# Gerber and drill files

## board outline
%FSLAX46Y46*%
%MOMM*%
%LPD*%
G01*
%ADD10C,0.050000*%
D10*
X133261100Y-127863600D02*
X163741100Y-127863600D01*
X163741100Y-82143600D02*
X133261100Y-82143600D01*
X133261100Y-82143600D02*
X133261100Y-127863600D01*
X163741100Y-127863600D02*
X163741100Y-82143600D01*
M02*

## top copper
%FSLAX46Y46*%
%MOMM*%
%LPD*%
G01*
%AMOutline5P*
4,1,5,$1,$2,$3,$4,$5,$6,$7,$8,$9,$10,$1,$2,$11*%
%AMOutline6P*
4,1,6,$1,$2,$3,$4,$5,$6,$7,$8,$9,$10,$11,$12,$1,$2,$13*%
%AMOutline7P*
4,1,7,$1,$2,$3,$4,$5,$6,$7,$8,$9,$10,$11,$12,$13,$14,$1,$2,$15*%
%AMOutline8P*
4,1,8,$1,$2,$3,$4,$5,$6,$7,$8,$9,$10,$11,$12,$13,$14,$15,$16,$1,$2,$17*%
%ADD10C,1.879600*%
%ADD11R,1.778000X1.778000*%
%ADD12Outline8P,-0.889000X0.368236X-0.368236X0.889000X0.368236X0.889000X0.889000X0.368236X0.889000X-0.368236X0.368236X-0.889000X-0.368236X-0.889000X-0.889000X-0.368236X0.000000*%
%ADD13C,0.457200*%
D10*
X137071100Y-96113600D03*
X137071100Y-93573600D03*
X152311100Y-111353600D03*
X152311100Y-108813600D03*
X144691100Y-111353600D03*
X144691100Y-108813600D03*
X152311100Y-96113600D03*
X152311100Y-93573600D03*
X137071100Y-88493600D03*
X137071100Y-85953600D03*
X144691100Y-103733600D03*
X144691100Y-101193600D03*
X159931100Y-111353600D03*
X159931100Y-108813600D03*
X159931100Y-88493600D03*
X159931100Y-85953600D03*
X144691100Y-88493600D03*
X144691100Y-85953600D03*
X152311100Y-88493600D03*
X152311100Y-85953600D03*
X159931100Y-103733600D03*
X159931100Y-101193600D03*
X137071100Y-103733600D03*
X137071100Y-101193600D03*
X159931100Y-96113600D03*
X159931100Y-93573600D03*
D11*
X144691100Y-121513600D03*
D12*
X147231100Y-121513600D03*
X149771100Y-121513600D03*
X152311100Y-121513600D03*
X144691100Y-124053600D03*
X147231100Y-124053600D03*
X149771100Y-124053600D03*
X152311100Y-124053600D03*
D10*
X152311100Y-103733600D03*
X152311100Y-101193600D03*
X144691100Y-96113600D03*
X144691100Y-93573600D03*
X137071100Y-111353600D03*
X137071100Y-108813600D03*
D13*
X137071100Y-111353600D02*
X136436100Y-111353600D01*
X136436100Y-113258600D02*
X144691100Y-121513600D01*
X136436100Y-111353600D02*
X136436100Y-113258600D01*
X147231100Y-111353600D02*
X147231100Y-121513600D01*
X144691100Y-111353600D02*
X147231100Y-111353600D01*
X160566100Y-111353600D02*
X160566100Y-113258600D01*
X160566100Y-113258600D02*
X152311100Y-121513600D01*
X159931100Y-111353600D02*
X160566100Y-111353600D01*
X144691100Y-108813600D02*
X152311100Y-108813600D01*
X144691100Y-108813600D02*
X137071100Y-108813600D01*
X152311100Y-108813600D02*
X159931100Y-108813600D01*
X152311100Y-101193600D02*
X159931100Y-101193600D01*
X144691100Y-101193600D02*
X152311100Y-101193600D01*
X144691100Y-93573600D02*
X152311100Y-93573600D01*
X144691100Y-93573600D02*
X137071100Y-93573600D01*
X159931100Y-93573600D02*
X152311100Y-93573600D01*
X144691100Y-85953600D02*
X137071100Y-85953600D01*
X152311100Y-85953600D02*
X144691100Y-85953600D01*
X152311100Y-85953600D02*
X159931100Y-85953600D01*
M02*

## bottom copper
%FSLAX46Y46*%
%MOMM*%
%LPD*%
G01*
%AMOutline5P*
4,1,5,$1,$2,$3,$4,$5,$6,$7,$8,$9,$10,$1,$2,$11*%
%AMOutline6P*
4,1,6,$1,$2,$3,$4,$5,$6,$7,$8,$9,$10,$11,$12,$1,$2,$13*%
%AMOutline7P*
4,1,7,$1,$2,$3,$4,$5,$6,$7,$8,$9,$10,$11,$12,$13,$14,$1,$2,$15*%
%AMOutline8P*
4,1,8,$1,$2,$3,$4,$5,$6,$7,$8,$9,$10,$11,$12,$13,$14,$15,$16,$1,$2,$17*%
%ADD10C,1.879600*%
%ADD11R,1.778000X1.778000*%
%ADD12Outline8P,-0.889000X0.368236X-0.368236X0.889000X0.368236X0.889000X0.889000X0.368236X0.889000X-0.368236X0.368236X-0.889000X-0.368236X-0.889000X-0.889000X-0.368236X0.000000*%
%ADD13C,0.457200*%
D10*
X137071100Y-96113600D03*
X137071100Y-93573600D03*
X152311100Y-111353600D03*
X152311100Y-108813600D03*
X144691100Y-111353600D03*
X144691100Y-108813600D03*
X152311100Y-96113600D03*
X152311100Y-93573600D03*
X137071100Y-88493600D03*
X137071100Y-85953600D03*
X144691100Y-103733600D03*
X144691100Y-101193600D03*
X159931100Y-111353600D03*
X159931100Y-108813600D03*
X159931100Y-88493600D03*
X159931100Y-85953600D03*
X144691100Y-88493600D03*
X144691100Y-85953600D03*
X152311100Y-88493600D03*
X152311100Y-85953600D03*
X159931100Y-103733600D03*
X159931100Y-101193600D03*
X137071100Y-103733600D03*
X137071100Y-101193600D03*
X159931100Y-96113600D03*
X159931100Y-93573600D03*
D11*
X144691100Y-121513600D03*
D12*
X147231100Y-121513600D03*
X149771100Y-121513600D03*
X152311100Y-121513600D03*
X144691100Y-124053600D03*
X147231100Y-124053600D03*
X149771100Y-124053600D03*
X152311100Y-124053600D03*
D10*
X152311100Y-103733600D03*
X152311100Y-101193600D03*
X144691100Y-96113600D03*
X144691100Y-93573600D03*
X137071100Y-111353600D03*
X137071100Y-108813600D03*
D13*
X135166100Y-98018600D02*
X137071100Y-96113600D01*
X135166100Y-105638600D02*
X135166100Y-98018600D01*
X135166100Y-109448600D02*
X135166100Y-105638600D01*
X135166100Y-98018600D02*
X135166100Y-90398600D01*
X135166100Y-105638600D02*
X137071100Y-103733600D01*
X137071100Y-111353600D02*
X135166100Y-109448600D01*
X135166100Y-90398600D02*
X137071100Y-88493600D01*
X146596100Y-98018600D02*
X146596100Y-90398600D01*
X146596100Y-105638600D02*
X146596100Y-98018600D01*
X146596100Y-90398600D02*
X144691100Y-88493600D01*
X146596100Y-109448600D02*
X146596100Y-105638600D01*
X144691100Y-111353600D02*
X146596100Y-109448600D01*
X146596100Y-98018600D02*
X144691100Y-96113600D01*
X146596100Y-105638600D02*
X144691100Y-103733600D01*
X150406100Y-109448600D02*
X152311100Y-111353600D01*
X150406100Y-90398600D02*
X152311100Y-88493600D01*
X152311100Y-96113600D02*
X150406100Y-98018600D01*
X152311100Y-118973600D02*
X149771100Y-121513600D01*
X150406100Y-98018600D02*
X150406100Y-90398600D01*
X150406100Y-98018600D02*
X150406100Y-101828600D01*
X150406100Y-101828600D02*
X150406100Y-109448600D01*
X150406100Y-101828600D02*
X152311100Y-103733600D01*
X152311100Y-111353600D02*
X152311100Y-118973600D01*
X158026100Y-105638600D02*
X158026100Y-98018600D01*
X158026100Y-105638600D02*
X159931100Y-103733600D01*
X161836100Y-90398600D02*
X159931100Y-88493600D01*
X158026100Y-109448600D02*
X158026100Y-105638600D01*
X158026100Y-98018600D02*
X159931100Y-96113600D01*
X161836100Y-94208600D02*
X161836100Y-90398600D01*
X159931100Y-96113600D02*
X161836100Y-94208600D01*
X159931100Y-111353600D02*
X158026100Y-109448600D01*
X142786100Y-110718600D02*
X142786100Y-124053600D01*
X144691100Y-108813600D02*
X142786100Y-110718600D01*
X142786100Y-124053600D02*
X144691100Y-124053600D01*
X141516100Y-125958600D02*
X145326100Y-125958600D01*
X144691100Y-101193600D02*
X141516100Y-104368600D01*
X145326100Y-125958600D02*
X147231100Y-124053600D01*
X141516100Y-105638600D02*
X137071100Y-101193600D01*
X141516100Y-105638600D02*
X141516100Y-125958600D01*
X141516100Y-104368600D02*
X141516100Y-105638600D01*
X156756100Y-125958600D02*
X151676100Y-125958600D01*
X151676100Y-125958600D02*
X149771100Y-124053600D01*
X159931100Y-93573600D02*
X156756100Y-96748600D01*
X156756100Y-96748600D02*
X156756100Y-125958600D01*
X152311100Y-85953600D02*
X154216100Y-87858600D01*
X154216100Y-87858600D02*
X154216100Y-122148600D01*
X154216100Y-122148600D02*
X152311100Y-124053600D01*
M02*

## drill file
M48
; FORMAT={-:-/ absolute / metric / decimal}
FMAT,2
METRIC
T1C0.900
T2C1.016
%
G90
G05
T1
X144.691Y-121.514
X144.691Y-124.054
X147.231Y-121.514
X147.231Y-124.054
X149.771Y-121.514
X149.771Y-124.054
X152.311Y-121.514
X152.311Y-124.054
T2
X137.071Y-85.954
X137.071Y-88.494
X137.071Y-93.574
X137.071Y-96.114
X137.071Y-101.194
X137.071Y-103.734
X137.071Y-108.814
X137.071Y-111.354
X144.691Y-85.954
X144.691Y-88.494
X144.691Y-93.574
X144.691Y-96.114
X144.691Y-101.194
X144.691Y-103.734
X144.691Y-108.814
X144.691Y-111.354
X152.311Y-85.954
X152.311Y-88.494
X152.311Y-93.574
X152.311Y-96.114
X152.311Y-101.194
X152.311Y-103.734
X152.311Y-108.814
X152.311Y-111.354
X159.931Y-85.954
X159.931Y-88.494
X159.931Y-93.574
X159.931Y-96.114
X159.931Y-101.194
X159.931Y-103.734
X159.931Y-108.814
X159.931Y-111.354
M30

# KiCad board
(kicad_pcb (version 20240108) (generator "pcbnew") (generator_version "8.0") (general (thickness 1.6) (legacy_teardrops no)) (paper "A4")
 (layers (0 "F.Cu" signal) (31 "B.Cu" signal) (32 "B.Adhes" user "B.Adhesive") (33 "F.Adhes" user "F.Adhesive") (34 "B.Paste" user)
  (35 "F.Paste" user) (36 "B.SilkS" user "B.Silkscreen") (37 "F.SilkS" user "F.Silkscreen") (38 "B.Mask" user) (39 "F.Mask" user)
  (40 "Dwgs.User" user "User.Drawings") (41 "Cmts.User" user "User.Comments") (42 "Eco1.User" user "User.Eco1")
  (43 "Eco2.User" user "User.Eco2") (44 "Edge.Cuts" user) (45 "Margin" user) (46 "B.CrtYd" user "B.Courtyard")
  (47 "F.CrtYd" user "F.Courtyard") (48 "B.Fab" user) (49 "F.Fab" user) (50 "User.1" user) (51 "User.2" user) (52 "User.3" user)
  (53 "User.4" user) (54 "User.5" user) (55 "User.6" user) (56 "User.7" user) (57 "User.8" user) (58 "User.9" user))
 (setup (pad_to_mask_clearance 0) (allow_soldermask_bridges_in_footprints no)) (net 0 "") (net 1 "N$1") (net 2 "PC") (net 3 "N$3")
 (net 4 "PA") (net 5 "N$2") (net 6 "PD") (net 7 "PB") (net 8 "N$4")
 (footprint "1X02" (layer "F.Cu") (at 137.0711 96.1136 90)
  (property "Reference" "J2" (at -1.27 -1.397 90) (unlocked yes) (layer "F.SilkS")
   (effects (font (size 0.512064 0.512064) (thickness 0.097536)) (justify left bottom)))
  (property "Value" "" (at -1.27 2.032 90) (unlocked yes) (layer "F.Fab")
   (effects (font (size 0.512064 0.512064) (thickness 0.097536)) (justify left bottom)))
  (pad "1" thru_hole circle (at 0 0 180) (size 1.8796 1.8796) (drill 1.016) (layers "*.Cu" "*.Mask") (remove_unused_layers no) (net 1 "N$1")
   (solder_mask_margin 0.1016) (thermal_bridge_angle 0))
  (pad "2" thru_hole circle (at 2.54 0 180) (size 1.8796 1.8796) (drill 1.016) (layers "*.Cu" "*.Mask") (remove_unused_layers no)
   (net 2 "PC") (solder_mask_margin 0.1016) (thermal_bridge_angle 0)))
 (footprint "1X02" (layer "F.Cu") (at 152.3111 111.3536 90)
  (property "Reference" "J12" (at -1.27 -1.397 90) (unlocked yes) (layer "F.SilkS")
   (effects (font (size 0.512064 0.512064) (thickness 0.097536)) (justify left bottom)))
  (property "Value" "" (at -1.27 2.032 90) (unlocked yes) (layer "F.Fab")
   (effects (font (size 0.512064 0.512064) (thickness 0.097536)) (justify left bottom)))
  (pad "1" thru_hole circle (at 0 0 180) (size 1.8796 1.8796) (drill 1.016) (layers "*.Cu" "*.Mask") (remove_unused_layers no) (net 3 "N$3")
   (solder_mask_margin 0.1016) (thermal_bridge_angle 0))
  (pad "2" thru_hole circle (at 2.54 0 180) (size 1.8796 1.8796) (drill 1.016) (layers "*.Cu" "*.Mask") (remove_unused_layers no)
   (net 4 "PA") (solder_mask_margin 0.1016) (thermal_bridge_angle 0)))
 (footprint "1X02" (layer "F.Cu") (at 144.6911 111.3536 90)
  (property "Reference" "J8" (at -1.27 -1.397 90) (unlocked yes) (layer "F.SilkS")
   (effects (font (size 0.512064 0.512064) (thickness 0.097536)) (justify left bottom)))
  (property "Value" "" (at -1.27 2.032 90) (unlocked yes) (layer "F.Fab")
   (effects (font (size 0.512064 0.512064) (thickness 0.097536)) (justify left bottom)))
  (pad "1" thru_hole circle (at 0 0 180) (size 1.8796 1.8796) (drill 1.016) (layers "*.Cu" "*.Mask") (remove_unused_layers no) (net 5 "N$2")
   (solder_mask_margin 0.1016) (thermal_bridge_angle 0))
  (pad "2" thru_hole circle (at 2.54 0 180) (size 1.8796 1.8796) (drill 1.016) (layers "*.Cu" "*.Mask") (remove_unused_layers no)
   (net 4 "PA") (solder_mask_margin 0.1016) (thermal_bridge_angle 0)))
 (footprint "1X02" (layer "F.Cu") (at 152.3111 96.1136 90)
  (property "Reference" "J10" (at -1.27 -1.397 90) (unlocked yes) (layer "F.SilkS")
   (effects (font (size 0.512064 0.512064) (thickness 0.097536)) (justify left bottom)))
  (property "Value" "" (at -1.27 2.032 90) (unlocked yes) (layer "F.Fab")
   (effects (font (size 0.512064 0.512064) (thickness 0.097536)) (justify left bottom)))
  (pad "1" thru_hole circle (at 0 0 180) (size 1.8796 1.8796) (drill 1.016) (layers "*.Cu" "*.Mask") (remove_unused_layers no) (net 3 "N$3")
   (solder_mask_margin 0.1016) (thermal_bridge_angle 0))
  (pad "2" thru_hole circle (at 2.54 0 180) (size 1.8796 1.8796) (drill 1.016) (layers "*.Cu" "*.Mask") (remove_unused_layers no)
   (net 2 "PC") (solder_mask_margin 0.1016) (thermal_bridge_angle 0)))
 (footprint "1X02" (layer "F.Cu") (at 137.0711 88.4936 90)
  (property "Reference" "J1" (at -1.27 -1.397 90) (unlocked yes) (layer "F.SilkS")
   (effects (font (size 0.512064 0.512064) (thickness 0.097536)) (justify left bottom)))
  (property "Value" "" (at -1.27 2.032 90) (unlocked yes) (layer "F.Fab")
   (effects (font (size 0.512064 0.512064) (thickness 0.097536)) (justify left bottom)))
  (pad "1" thru_hole circle (at 0 0 180) (size 1.8796 1.8796) (drill 1.016) (layers "*.Cu" "*.Mask") (remove_unused_layers no) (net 1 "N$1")
   (solder_mask_margin 0.1016) (thermal_bridge_angle 0))
  (pad "2" thru_hole circle (at 2.54 0 180) (size 1.8796 1.8796) (drill 1.016) (layers "*.Cu" "*.Mask") (remove_unused_layers no)
   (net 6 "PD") (solder_mask_margin 0.1016) (thermal_bridge_angle 0)))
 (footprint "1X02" (layer "F.Cu") (at 144.6911 103.7336 90)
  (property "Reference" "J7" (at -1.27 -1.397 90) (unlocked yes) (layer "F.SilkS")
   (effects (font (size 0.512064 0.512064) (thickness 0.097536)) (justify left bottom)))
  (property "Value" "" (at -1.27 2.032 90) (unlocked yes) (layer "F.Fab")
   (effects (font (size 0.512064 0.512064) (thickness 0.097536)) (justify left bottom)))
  (pad "1" thru_hole circle (at 0 0 180) (size 1.8796 1.8796) (drill 1.016) (layers "*.Cu" "*.Mask") (remove_unused_layers no) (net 5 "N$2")
   (solder_mask_margin 0.1016) (thermal_bridge_angle 0))
  (pad "2" thru_hole circle (at 2.54 0 180) (size 1.8796 1.8796) (drill 1.016) (layers "*.Cu" "*.Mask") (remove_unused_layers no)
   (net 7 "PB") (solder_mask_margin 0.1016) (thermal_bridge_angle 0)))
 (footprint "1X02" (layer "F.Cu") (at 159.9311 111.3536 90)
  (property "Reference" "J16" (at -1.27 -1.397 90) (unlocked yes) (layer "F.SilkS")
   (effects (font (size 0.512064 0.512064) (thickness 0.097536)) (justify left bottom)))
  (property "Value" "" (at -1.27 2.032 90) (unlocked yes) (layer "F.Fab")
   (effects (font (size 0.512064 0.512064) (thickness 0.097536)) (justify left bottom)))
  (pad "1" thru_hole circle (at 0 0 180) (size 1.8796 1.8796) (drill 1.016) (layers "*.Cu" "*.Mask") (remove_unused_layers no) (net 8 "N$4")
   (solder_mask_margin 0.1016) (thermal_bridge_angle 0))
  (pad "2" thru_hole circle (at 2.54 0 180) (size 1.8796 1.8796) (drill 1.016) (layers "*.Cu" "*.Mask") (remove_unused_layers no)
   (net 4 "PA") (solder_mask_margin 0.1016) (thermal_bridge_angle 0)))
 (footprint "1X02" (layer "F.Cu") (at 159.9311 88.4936 90)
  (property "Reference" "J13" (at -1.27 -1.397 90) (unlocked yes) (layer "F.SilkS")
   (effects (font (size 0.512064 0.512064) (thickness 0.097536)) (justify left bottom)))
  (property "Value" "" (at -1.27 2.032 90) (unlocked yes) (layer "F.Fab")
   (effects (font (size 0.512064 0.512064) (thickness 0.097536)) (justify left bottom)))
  (pad "1" thru_hole circle (at 0 0 180) (size 1.8796 1.8796) (drill 1.016) (layers "*.Cu" "*.Mask") (remove_unused_layers no) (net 8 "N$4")
   (solder_mask_margin 0.1016) (thermal_bridge_angle 0))
  (pad "2" thru_hole circle (at 2.54 0 180) (size 1.8796 1.8796) (drill 1.016) (layers "*.Cu" "*.Mask") (remove_unused_layers no)
   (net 6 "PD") (solder_mask_margin 0.1016) (thermal_bridge_angle 0)))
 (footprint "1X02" (layer "F.Cu") (at 144.6911 88.4936 90)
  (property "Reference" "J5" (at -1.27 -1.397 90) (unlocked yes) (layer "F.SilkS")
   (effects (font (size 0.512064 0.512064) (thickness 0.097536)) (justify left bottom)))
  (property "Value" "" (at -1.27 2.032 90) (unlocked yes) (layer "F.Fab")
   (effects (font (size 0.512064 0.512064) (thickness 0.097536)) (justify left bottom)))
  (pad "1" thru_hole circle (at 0 0 180) (size 1.8796 1.8796) (drill 1.016) (layers "*.Cu" "*.Mask") (remove_unused_layers no) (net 5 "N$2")
   (solder_mask_margin 0.1016) (thermal_bridge_angle 0))
  (pad "2" thru_hole circle (at 2.54 0 180) (size 1.8796 1.8796) (drill 1.016) (layers "*.Cu" "*.Mask") (remove_unused_layers no)
   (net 6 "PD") (solder_mask_margin 0.1016) (thermal_bridge_angle 0)))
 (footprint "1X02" (layer "F.Cu") (at 152.3111 88.4936 90)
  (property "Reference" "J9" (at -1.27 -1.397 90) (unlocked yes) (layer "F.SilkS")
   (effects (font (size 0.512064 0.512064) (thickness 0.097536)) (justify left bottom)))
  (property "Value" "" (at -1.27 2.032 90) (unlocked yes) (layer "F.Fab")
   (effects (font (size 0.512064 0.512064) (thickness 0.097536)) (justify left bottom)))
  (pad "1" thru_hole circle (at 0 0 180) (size 1.8796 1.8796) (drill 1.016) (layers "*.Cu" "*.Mask") (remove_unused_layers no) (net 3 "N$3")
   (solder_mask_margin 0.1016) (thermal_bridge_angle 0))
  (pad "2" thru_hole circle (at 2.54 0 180) (size 1.8796 1.8796) (drill 1.016) (layers "*.Cu" "*.Mask") (remove_unused_layers no)
   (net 6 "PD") (solder_mask_margin 0.1016) (thermal_bridge_angle 0)))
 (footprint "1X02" (layer "F.Cu") (at 159.9311 103.7336 90)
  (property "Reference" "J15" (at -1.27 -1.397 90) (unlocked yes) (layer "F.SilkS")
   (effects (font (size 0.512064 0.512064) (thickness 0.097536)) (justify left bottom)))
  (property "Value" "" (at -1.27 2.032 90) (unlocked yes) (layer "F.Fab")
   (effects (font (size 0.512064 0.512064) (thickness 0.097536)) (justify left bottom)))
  (pad "1" thru_hole circle (at 0 0 180) (size 1.8796 1.8796) (drill 1.016) (layers "*.Cu" "*.Mask") (remove_unused_layers no) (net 8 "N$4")
   (solder_mask_margin 0.1016) (thermal_bridge_angle 0))
  (pad "2" thru_hole circle (at 2.54 0 180) (size 1.8796 1.8796) (drill 1.016) (layers "*.Cu" "*.Mask") (remove_unused_layers no)
   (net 7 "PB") (solder_mask_margin 0.1016) (thermal_bridge_angle 0)))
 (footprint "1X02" (layer "F.Cu") (at 137.0711 103.7336 90)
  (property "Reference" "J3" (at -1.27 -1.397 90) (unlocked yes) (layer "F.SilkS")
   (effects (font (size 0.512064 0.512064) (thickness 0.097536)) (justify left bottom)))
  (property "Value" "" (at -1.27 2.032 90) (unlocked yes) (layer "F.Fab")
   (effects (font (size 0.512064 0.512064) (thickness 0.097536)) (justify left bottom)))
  (pad "1" thru_hole circle (at 0 0 180) (size 1.8796 1.8796) (drill 1.016) (layers "*.Cu" "*.Mask") (remove_unused_layers no) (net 1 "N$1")
   (solder_mask_margin 0.1016) (thermal_bridge_angle 0))
  (pad "2" thru_hole circle (at 2.54 0 180) (size 1.8796 1.8796) (drill 1.016) (layers "*.Cu" "*.Mask") (remove_unused_layers no)
   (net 7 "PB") (solder_mask_margin 0.1016) (thermal_bridge_angle 0)))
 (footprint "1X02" (layer "F.Cu") (at 159.9311 96.1136 90)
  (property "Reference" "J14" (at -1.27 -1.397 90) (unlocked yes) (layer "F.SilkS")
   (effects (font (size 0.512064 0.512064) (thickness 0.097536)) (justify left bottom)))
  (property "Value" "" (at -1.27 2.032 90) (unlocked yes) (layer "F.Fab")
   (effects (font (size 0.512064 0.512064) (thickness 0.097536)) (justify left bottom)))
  (pad "1" thru_hole circle (at 0 0 180) (size 1.8796 1.8796) (drill 1.016) (layers "*.Cu" "*.Mask") (remove_unused_layers no) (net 8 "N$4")
   (solder_mask_margin 0.1016) (thermal_bridge_angle 0))
  (pad "2" thru_hole circle (at 2.54 0 180) (size 1.8796 1.8796) (drill 1.016) (layers "*.Cu" "*.Mask") (remove_unused_layers no)
   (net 2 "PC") (solder_mask_margin 0.1016) (thermal_bridge_angle 0)))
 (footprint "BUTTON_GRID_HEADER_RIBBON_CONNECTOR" (layer "F.Cu") (at 148.5011 122.7836)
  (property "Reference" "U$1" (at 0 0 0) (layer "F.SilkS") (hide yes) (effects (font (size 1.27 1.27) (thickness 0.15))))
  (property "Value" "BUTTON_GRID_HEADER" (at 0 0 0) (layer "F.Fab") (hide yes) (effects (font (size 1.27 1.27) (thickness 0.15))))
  (pad "P1" thru_hole rect (at -3.81 -1.27) (size 1.778 1.778) (drill 0.9) (layers "*.Cu" "*.Mask") (remove_unused_layers no) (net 1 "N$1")
   (solder_mask_margin 0.1016) (thermal_bridge_angle 0))
  (pad "P2" thru_hole roundrect (at -1.27 -1.27) (size 1.778 1.778) (drill 0.9) (layers "*.Cu" "*.Mask") (remove_unused_layers no)
   (roundrect_rratio 0.25) (chamfer_ratio 0.2928932188) (chamfer top_left top_right bottom_left bottom_right) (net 5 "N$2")
   (solder_mask_margin 0.1016) (thermal_bridge_angle 0))
  (pad "P3" thru_hole roundrect (at 1.27 -1.27) (size 1.778 1.778) (drill 0.9) (layers "*.Cu" "*.Mask") (remove_unused_layers no)
   (roundrect_rratio 0.25) (chamfer_ratio 0.2928932188) (chamfer top_left top_right bottom_left bottom_right) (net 3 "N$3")
   (solder_mask_margin 0.1016) (thermal_bridge_angle 0))
  (pad "P4" thru_hole roundrect (at 3.81 -1.27) (size 1.778 1.778) (drill 0.9) (layers "*.Cu" "*.Mask") (remove_unused_layers no)
   (roundrect_rratio 0.25) (chamfer_ratio 0.2928932188) (chamfer top_left top_right bottom_left bottom_right) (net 8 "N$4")
   (solder_mask_margin 0.1016) (thermal_bridge_angle 0))
  (pad "PA" thru_hole roundrect (at -3.81 1.27) (size 1.778 1.778) (drill 0.9) (layers "*.Cu" "*.Mask") (remove_unused_layers no)
   (roundrect_rratio 0.25) (chamfer_ratio 0.2928932188) (chamfer top_left top_right bottom_left bottom_right) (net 4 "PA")
   (solder_mask_margin 0.1016) (thermal_bridge_angle 0))
  (pad "PB" thru_hole roundrect (at -1.27 1.27) (size 1.778 1.778) (drill 0.9) (layers "*.Cu" "*.Mask") (remove_unused_layers no)
   (roundrect_rratio 0.25) (chamfer_ratio 0.2928932188) (chamfer top_left top_right bottom_left bottom_right) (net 7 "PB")
   (solder_mask_margin 0.1016) (thermal_bridge_angle 0))
  (pad "PC" thru_hole roundrect (at 1.27 1.27) (size 1.778 1.778) (drill 0.9) (layers "*.Cu" "*.Mask") (remove_unused_layers no)
   (roundrect_rratio 0.25) (chamfer_ratio 0.2928932188) (chamfer top_left top_right bottom_left bottom_right) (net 2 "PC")
   (solder_mask_margin 0.1016) (thermal_bridge_angle 0))
  (pad "PD" thru_hole roundrect (at 3.81 1.27) (size 1.778 1.778) (drill 0.9) (layers "*.Cu" "*.Mask") (remove_unused_layers no)
   (roundrect_rratio 0.25) (chamfer_ratio 0.2928932188) (chamfer top_left top_right bottom_left bottom_right) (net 6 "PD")
   (solder_mask_margin 0.1016) (thermal_bridge_angle 0)))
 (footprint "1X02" (layer "F.Cu") (at 152.3111 103.7336 90)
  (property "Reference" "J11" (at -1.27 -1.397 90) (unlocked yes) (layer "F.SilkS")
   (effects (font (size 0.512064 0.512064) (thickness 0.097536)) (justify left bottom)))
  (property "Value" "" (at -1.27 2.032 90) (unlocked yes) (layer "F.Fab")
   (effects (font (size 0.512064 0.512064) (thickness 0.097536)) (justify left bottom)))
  (pad "1" thru_hole circle (at 0 0 180) (size 1.8796 1.8796) (drill 1.016) (layers "*.Cu" "*.Mask") (remove_unused_layers no) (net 3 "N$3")
   (solder_mask_margin 0.1016) (thermal_bridge_angle 0))
  (pad "2" thru_hole circle (at 2.54 0 180) (size 1.8796 1.8796) (drill 1.016) (layers "*.Cu" "*.Mask") (remove_unused_layers no)
   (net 7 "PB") (solder_mask_margin 0.1016) (thermal_bridge_angle 0)))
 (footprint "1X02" (layer "F.Cu") (at 144.6911 96.1136 90)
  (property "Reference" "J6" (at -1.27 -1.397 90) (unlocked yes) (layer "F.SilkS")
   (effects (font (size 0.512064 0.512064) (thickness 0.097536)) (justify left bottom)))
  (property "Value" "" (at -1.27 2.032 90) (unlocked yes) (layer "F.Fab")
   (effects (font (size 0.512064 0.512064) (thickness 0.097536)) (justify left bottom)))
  (pad "1" thru_hole circle (at 0 0 180) (size 1.8796 1.8796) (drill 1.016) (layers "*.Cu" "*.Mask") (remove_unused_layers no) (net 5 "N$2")
   (solder_mask_margin 0.1016) (thermal_bridge_angle 0))
  (pad "2" thru_hole circle (at 2.54 0 180) (size 1.8796 1.8796) (drill 1.016) (layers "*.Cu" "*.Mask") (remove_unused_layers no)
   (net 2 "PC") (solder_mask_margin 0.1016) (thermal_bridge_angle 0)))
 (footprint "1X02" (layer "F.Cu") (at 137.0711 111.3536 90)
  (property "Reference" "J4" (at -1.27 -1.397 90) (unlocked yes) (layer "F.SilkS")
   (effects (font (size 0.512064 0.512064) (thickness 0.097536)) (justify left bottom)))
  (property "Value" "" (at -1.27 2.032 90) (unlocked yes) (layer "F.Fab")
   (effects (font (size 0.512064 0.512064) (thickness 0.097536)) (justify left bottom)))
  (pad "1" thru_hole circle (at 0 0 180) (size 1.8796 1.8796) (drill 1.016) (layers "*.Cu" "*.Mask") (remove_unused_layers no) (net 1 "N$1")
   (solder_mask_margin 0.1016) (thermal_bridge_angle 0))
  (pad "2" thru_hole circle (at 2.54 0 180) (size 1.8796 1.8796) (drill 1.016) (layers "*.Cu" "*.Mask") (remove_unused_layers no)
   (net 4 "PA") (solder_mask_margin 0.1016) (thermal_bridge_angle 0)))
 (gr_line (start 133.2611 127.8636) (end 163.7411 127.8636) (stroke (width 0.05) (type solid)) (layer "Edge.Cuts"))
 (gr_line (start 163.7411 82.1436) (end 133.2611 82.1436) (stroke (width 0.05) (type solid)) (layer "Edge.Cuts"))
 (gr_line (start 133.2611 82.1436) (end 133.2611 127.8636) (stroke (width 0.05) (type solid)) (layer "Edge.Cuts"))
 (gr_line (start 163.7411 127.8636) (end 163.7411 82.1436) (stroke (width 0.05) (type solid)) (layer "Edge.Cuts"))
 (segment (start 137.0711 111.3536) (end 136.4361 111.3536) (width 0.4572) (layer "F.Cu") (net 1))
 (segment (start 136.4361 113.2586) (end 144.6911 121.5136) (width 0.4572) (layer "F.Cu") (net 1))
 (segment (start 136.4361 111.3536) (end 136.4361 113.2586) (width 0.4572) (layer "F.Cu") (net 1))
 (segment (start 135.1661 98.0186) (end 137.0711 96.1136) (width 0.4572) (layer "B.Cu") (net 1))
 (segment (start 135.1661 105.6386) (end 135.1661 98.0186) (width 0.4572) (layer "B.Cu") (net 1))
 (segment (start 135.1661 109.4486) (end 135.1661 105.6386) (width 0.4572) (layer "B.Cu") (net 1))
 (segment (start 135.1661 98.0186) (end 135.1661 90.3986) (width 0.4572) (layer "B.Cu") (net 1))
 (segment (start 135.1661 105.6386) (end 137.0711 103.7336) (width 0.4572) (layer "B.Cu") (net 1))
 (segment (start 137.0711 111.3536) (end 135.1661 109.4486) (width 0.4572) (layer "B.Cu") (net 1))
 (segment (start 135.1661 90.3986) (end 137.0711 88.4936) (width 0.4572) (layer "B.Cu") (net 1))
 (segment (start 147.2311 111.3536) (end 147.2311 121.5136) (width 0.4572) (layer "F.Cu") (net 5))
 (segment (start 144.6911 111.3536) (end 147.2311 111.3536) (width 0.4572) (layer "F.Cu") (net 5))
 (segment (start 146.5961 98.0186) (end 146.5961 90.3986) (width 0.4572) (layer "B.Cu") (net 5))
 (segment (start 146.5961 105.6386) (end 146.5961 98.0186) (width 0.4572) (layer "B.Cu") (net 5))
 (segment (start 146.5961 90.3986) (end 144.6911 88.4936) (width 0.4572) (layer "B.Cu") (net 5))
 (segment (start 146.5961 109.4486) (end 146.5961 105.6386) (width 0.4572) (layer "B.Cu") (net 5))
 (segment (start 144.6911 111.3536) (end 146.5961 109.4486) (width 0.4572) (layer "B.Cu") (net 5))
 (segment (start 146.5961 98.0186) (end 144.6911 96.1136) (width 0.4572) (layer "B.Cu") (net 5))
 (segment (start 146.5961 105.6386) (end 144.6911 103.7336) (width 0.4572) (layer "B.Cu") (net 5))
 (segment (start 150.4061 109.4486) (end 152.3111 111.3536) (width 0.4572) (layer "B.Cu") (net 3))
 (segment (start 150.4061 90.3986) (end 152.3111 88.4936) (width 0.4572) (layer "B.Cu") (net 3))
 (segment (start 152.3111 96.1136) (end 150.4061 98.0186) (width 0.4572) (layer "B.Cu") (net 3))
 (segment (start 152.3111 118.9736) (end 149.7711 121.5136) (width 0.4572) (layer "B.Cu") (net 3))
 (segment (start 150.4061 98.0186) (end 150.4061 90.3986) (width 0.4572) (layer "B.Cu") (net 3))
 (segment (start 150.4061 98.0186) (end 150.4061 101.8286) (width 0.4572) (layer "B.Cu") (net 3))
 (segment (start 150.4061 101.8286) (end 150.4061 109.4486) (width 0.4572) (layer "B.Cu") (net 3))
 (segment (start 150.4061 101.8286) (end 152.3111 103.7336) (width 0.4572) (layer "B.Cu") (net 3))
 (segment (start 152.3111 111.3536) (end 152.3111 118.9736) (width 0.4572) (layer "B.Cu") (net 3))
 (segment (start 160.5661 111.3536) (end 160.5661 113.2586) (width 0.4572) (layer "F.Cu") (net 8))
 (segment (start 160.5661 113.2586) (end 152.3111 121.5136) (width 0.4572) (layer "F.Cu") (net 8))
 (segment (start 159.9311 111.3536) (end 160.5661 111.3536) (width 0.4572) (layer "F.Cu") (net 8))
 (segment (start 158.0261 105.6386) (end 158.0261 98.0186) (width 0.4572) (layer "B.Cu") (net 8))
 (segment (start 158.0261 105.6386) (end 159.9311 103.7336) (width 0.4572) (layer "B.Cu") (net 8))
 (segment (start 161.8361 90.3986) (end 159.9311 88.4936) (width 0.4572) (layer "B.Cu") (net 8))
 (segment (start 158.0261 109.4486) (end 158.0261 105.6386) (width 0.4572) (layer "B.Cu") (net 8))
 (segment (start 158.0261 98.0186) (end 159.9311 96.1136) (width 0.4572) (layer "B.Cu") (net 8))
 (segment (start 161.8361 94.2086) (end 161.8361 90.3986) (width 0.4572) (layer "B.Cu") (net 8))
 (segment (start 159.9311 96.1136) (end 161.8361 94.2086) (width 0.4572) (layer "B.Cu") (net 8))
 (segment (start 159.9311 111.3536) (end 158.0261 109.4486) (width 0.4572) (layer "B.Cu") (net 8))
 (segment (start 144.6911 108.8136) (end 152.3111 108.8136) (width 0.4572) (layer "F.Cu") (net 4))
 (segment (start 144.6911 108.8136) (end 137.0711 108.8136) (width 0.4572) (layer "F.Cu") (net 4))
 (segment (start 152.3111 108.8136) (end 159.9311 108.8136) (width 0.4572) (layer "F.Cu") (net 4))
 (segment (start 142.7861 110.7186) (end 142.7861 124.0536) (width 0.4572) (layer "B.Cu") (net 4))
 (segment (start 144.6911 108.8136) (end 142.7861 110.7186) (width 0.4572) (layer "B.Cu") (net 4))
 (segment (start 142.7861 124.0536) (end 144.6911 124.0536) (width 0.4572) (layer "B.Cu") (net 4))
 (segment (start 152.3111 101.1936) (end 159.9311 101.1936) (width 0.4572) (layer "F.Cu") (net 7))
 (segment (start 144.6911 101.1936) (end 152.3111 101.1936) (width 0.4572) (layer "F.Cu") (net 7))
 (segment (start 141.5161 125.9586) (end 145.3261 125.9586) (width 0.4572) (layer "B.Cu") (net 7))
 (segment (start 144.6911 101.1936) (end 141.5161 104.3686) (width 0.4572) (layer "B.Cu") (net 7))
 (segment (start 145.3261 125.9586) (end 147.2311 124.0536) (width 0.4572) (layer "B.Cu") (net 7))
 (segment (start 141.5161 105.6386) (end 137.0711 101.1936) (width 0.4572) (layer "B.Cu") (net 7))
 (segment (start 141.5161 105.6386) (end 141.5161 125.9586) (width 0.4572) (layer "B.Cu") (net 7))
 (segment (start 141.5161 104.3686) (end 141.5161 105.6386) (width 0.4572) (layer "B.Cu") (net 7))
 (segment (start 144.6911 93.5736) (end 152.3111 93.5736) (width 0.4572) (layer "F.Cu") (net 2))
 (segment (start 144.6911 93.5736) (end 137.0711 93.5736) (width 0.4572) (layer "F.Cu") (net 2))
 (segment (start 159.9311 93.5736) (end 152.3111 93.5736) (width 0.4572) (layer "F.Cu") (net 2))
 (segment (start 156.7561 125.9586) (end 151.6761 125.9586) (width 0.4572) (layer "B.Cu") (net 2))
 (segment (start 151.6761 125.9586) (end 149.7711 124.0536) (width 0.4572) (layer "B.Cu") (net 2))
 (segment (start 159.9311 93.5736) (end 156.7561 96.7486) (width 0.4572) (layer "B.Cu") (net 2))
 (segment (start 156.7561 96.7486) (end 156.7561 125.9586) (width 0.4572) (layer "B.Cu") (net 2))
 (segment (start 144.6911 85.9536) (end 137.0711 85.9536) (width 0.4572) (layer "F.Cu") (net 6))
 (segment (start 152.3111 85.9536) (end 144.6911 85.9536) (width 0.4572) (layer "F.Cu") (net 6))
 (segment (start 152.3111 85.9536) (end 159.9311 85.9536) (width 0.4572) (layer "F.Cu") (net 6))
 (segment (start 152.3111 85.9536) (end 154.2161 87.8586) (width 0.4572) (layer "B.Cu") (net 6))
 (segment (start 154.2161 87.8586) (end 154.2161 122.1486) (width 0.4572) (layer "B.Cu") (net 6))
 (segment (start 154.2161 122.1486) (end 152.3111 124.0536) (width 0.4572) (layer "B.Cu") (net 6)))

